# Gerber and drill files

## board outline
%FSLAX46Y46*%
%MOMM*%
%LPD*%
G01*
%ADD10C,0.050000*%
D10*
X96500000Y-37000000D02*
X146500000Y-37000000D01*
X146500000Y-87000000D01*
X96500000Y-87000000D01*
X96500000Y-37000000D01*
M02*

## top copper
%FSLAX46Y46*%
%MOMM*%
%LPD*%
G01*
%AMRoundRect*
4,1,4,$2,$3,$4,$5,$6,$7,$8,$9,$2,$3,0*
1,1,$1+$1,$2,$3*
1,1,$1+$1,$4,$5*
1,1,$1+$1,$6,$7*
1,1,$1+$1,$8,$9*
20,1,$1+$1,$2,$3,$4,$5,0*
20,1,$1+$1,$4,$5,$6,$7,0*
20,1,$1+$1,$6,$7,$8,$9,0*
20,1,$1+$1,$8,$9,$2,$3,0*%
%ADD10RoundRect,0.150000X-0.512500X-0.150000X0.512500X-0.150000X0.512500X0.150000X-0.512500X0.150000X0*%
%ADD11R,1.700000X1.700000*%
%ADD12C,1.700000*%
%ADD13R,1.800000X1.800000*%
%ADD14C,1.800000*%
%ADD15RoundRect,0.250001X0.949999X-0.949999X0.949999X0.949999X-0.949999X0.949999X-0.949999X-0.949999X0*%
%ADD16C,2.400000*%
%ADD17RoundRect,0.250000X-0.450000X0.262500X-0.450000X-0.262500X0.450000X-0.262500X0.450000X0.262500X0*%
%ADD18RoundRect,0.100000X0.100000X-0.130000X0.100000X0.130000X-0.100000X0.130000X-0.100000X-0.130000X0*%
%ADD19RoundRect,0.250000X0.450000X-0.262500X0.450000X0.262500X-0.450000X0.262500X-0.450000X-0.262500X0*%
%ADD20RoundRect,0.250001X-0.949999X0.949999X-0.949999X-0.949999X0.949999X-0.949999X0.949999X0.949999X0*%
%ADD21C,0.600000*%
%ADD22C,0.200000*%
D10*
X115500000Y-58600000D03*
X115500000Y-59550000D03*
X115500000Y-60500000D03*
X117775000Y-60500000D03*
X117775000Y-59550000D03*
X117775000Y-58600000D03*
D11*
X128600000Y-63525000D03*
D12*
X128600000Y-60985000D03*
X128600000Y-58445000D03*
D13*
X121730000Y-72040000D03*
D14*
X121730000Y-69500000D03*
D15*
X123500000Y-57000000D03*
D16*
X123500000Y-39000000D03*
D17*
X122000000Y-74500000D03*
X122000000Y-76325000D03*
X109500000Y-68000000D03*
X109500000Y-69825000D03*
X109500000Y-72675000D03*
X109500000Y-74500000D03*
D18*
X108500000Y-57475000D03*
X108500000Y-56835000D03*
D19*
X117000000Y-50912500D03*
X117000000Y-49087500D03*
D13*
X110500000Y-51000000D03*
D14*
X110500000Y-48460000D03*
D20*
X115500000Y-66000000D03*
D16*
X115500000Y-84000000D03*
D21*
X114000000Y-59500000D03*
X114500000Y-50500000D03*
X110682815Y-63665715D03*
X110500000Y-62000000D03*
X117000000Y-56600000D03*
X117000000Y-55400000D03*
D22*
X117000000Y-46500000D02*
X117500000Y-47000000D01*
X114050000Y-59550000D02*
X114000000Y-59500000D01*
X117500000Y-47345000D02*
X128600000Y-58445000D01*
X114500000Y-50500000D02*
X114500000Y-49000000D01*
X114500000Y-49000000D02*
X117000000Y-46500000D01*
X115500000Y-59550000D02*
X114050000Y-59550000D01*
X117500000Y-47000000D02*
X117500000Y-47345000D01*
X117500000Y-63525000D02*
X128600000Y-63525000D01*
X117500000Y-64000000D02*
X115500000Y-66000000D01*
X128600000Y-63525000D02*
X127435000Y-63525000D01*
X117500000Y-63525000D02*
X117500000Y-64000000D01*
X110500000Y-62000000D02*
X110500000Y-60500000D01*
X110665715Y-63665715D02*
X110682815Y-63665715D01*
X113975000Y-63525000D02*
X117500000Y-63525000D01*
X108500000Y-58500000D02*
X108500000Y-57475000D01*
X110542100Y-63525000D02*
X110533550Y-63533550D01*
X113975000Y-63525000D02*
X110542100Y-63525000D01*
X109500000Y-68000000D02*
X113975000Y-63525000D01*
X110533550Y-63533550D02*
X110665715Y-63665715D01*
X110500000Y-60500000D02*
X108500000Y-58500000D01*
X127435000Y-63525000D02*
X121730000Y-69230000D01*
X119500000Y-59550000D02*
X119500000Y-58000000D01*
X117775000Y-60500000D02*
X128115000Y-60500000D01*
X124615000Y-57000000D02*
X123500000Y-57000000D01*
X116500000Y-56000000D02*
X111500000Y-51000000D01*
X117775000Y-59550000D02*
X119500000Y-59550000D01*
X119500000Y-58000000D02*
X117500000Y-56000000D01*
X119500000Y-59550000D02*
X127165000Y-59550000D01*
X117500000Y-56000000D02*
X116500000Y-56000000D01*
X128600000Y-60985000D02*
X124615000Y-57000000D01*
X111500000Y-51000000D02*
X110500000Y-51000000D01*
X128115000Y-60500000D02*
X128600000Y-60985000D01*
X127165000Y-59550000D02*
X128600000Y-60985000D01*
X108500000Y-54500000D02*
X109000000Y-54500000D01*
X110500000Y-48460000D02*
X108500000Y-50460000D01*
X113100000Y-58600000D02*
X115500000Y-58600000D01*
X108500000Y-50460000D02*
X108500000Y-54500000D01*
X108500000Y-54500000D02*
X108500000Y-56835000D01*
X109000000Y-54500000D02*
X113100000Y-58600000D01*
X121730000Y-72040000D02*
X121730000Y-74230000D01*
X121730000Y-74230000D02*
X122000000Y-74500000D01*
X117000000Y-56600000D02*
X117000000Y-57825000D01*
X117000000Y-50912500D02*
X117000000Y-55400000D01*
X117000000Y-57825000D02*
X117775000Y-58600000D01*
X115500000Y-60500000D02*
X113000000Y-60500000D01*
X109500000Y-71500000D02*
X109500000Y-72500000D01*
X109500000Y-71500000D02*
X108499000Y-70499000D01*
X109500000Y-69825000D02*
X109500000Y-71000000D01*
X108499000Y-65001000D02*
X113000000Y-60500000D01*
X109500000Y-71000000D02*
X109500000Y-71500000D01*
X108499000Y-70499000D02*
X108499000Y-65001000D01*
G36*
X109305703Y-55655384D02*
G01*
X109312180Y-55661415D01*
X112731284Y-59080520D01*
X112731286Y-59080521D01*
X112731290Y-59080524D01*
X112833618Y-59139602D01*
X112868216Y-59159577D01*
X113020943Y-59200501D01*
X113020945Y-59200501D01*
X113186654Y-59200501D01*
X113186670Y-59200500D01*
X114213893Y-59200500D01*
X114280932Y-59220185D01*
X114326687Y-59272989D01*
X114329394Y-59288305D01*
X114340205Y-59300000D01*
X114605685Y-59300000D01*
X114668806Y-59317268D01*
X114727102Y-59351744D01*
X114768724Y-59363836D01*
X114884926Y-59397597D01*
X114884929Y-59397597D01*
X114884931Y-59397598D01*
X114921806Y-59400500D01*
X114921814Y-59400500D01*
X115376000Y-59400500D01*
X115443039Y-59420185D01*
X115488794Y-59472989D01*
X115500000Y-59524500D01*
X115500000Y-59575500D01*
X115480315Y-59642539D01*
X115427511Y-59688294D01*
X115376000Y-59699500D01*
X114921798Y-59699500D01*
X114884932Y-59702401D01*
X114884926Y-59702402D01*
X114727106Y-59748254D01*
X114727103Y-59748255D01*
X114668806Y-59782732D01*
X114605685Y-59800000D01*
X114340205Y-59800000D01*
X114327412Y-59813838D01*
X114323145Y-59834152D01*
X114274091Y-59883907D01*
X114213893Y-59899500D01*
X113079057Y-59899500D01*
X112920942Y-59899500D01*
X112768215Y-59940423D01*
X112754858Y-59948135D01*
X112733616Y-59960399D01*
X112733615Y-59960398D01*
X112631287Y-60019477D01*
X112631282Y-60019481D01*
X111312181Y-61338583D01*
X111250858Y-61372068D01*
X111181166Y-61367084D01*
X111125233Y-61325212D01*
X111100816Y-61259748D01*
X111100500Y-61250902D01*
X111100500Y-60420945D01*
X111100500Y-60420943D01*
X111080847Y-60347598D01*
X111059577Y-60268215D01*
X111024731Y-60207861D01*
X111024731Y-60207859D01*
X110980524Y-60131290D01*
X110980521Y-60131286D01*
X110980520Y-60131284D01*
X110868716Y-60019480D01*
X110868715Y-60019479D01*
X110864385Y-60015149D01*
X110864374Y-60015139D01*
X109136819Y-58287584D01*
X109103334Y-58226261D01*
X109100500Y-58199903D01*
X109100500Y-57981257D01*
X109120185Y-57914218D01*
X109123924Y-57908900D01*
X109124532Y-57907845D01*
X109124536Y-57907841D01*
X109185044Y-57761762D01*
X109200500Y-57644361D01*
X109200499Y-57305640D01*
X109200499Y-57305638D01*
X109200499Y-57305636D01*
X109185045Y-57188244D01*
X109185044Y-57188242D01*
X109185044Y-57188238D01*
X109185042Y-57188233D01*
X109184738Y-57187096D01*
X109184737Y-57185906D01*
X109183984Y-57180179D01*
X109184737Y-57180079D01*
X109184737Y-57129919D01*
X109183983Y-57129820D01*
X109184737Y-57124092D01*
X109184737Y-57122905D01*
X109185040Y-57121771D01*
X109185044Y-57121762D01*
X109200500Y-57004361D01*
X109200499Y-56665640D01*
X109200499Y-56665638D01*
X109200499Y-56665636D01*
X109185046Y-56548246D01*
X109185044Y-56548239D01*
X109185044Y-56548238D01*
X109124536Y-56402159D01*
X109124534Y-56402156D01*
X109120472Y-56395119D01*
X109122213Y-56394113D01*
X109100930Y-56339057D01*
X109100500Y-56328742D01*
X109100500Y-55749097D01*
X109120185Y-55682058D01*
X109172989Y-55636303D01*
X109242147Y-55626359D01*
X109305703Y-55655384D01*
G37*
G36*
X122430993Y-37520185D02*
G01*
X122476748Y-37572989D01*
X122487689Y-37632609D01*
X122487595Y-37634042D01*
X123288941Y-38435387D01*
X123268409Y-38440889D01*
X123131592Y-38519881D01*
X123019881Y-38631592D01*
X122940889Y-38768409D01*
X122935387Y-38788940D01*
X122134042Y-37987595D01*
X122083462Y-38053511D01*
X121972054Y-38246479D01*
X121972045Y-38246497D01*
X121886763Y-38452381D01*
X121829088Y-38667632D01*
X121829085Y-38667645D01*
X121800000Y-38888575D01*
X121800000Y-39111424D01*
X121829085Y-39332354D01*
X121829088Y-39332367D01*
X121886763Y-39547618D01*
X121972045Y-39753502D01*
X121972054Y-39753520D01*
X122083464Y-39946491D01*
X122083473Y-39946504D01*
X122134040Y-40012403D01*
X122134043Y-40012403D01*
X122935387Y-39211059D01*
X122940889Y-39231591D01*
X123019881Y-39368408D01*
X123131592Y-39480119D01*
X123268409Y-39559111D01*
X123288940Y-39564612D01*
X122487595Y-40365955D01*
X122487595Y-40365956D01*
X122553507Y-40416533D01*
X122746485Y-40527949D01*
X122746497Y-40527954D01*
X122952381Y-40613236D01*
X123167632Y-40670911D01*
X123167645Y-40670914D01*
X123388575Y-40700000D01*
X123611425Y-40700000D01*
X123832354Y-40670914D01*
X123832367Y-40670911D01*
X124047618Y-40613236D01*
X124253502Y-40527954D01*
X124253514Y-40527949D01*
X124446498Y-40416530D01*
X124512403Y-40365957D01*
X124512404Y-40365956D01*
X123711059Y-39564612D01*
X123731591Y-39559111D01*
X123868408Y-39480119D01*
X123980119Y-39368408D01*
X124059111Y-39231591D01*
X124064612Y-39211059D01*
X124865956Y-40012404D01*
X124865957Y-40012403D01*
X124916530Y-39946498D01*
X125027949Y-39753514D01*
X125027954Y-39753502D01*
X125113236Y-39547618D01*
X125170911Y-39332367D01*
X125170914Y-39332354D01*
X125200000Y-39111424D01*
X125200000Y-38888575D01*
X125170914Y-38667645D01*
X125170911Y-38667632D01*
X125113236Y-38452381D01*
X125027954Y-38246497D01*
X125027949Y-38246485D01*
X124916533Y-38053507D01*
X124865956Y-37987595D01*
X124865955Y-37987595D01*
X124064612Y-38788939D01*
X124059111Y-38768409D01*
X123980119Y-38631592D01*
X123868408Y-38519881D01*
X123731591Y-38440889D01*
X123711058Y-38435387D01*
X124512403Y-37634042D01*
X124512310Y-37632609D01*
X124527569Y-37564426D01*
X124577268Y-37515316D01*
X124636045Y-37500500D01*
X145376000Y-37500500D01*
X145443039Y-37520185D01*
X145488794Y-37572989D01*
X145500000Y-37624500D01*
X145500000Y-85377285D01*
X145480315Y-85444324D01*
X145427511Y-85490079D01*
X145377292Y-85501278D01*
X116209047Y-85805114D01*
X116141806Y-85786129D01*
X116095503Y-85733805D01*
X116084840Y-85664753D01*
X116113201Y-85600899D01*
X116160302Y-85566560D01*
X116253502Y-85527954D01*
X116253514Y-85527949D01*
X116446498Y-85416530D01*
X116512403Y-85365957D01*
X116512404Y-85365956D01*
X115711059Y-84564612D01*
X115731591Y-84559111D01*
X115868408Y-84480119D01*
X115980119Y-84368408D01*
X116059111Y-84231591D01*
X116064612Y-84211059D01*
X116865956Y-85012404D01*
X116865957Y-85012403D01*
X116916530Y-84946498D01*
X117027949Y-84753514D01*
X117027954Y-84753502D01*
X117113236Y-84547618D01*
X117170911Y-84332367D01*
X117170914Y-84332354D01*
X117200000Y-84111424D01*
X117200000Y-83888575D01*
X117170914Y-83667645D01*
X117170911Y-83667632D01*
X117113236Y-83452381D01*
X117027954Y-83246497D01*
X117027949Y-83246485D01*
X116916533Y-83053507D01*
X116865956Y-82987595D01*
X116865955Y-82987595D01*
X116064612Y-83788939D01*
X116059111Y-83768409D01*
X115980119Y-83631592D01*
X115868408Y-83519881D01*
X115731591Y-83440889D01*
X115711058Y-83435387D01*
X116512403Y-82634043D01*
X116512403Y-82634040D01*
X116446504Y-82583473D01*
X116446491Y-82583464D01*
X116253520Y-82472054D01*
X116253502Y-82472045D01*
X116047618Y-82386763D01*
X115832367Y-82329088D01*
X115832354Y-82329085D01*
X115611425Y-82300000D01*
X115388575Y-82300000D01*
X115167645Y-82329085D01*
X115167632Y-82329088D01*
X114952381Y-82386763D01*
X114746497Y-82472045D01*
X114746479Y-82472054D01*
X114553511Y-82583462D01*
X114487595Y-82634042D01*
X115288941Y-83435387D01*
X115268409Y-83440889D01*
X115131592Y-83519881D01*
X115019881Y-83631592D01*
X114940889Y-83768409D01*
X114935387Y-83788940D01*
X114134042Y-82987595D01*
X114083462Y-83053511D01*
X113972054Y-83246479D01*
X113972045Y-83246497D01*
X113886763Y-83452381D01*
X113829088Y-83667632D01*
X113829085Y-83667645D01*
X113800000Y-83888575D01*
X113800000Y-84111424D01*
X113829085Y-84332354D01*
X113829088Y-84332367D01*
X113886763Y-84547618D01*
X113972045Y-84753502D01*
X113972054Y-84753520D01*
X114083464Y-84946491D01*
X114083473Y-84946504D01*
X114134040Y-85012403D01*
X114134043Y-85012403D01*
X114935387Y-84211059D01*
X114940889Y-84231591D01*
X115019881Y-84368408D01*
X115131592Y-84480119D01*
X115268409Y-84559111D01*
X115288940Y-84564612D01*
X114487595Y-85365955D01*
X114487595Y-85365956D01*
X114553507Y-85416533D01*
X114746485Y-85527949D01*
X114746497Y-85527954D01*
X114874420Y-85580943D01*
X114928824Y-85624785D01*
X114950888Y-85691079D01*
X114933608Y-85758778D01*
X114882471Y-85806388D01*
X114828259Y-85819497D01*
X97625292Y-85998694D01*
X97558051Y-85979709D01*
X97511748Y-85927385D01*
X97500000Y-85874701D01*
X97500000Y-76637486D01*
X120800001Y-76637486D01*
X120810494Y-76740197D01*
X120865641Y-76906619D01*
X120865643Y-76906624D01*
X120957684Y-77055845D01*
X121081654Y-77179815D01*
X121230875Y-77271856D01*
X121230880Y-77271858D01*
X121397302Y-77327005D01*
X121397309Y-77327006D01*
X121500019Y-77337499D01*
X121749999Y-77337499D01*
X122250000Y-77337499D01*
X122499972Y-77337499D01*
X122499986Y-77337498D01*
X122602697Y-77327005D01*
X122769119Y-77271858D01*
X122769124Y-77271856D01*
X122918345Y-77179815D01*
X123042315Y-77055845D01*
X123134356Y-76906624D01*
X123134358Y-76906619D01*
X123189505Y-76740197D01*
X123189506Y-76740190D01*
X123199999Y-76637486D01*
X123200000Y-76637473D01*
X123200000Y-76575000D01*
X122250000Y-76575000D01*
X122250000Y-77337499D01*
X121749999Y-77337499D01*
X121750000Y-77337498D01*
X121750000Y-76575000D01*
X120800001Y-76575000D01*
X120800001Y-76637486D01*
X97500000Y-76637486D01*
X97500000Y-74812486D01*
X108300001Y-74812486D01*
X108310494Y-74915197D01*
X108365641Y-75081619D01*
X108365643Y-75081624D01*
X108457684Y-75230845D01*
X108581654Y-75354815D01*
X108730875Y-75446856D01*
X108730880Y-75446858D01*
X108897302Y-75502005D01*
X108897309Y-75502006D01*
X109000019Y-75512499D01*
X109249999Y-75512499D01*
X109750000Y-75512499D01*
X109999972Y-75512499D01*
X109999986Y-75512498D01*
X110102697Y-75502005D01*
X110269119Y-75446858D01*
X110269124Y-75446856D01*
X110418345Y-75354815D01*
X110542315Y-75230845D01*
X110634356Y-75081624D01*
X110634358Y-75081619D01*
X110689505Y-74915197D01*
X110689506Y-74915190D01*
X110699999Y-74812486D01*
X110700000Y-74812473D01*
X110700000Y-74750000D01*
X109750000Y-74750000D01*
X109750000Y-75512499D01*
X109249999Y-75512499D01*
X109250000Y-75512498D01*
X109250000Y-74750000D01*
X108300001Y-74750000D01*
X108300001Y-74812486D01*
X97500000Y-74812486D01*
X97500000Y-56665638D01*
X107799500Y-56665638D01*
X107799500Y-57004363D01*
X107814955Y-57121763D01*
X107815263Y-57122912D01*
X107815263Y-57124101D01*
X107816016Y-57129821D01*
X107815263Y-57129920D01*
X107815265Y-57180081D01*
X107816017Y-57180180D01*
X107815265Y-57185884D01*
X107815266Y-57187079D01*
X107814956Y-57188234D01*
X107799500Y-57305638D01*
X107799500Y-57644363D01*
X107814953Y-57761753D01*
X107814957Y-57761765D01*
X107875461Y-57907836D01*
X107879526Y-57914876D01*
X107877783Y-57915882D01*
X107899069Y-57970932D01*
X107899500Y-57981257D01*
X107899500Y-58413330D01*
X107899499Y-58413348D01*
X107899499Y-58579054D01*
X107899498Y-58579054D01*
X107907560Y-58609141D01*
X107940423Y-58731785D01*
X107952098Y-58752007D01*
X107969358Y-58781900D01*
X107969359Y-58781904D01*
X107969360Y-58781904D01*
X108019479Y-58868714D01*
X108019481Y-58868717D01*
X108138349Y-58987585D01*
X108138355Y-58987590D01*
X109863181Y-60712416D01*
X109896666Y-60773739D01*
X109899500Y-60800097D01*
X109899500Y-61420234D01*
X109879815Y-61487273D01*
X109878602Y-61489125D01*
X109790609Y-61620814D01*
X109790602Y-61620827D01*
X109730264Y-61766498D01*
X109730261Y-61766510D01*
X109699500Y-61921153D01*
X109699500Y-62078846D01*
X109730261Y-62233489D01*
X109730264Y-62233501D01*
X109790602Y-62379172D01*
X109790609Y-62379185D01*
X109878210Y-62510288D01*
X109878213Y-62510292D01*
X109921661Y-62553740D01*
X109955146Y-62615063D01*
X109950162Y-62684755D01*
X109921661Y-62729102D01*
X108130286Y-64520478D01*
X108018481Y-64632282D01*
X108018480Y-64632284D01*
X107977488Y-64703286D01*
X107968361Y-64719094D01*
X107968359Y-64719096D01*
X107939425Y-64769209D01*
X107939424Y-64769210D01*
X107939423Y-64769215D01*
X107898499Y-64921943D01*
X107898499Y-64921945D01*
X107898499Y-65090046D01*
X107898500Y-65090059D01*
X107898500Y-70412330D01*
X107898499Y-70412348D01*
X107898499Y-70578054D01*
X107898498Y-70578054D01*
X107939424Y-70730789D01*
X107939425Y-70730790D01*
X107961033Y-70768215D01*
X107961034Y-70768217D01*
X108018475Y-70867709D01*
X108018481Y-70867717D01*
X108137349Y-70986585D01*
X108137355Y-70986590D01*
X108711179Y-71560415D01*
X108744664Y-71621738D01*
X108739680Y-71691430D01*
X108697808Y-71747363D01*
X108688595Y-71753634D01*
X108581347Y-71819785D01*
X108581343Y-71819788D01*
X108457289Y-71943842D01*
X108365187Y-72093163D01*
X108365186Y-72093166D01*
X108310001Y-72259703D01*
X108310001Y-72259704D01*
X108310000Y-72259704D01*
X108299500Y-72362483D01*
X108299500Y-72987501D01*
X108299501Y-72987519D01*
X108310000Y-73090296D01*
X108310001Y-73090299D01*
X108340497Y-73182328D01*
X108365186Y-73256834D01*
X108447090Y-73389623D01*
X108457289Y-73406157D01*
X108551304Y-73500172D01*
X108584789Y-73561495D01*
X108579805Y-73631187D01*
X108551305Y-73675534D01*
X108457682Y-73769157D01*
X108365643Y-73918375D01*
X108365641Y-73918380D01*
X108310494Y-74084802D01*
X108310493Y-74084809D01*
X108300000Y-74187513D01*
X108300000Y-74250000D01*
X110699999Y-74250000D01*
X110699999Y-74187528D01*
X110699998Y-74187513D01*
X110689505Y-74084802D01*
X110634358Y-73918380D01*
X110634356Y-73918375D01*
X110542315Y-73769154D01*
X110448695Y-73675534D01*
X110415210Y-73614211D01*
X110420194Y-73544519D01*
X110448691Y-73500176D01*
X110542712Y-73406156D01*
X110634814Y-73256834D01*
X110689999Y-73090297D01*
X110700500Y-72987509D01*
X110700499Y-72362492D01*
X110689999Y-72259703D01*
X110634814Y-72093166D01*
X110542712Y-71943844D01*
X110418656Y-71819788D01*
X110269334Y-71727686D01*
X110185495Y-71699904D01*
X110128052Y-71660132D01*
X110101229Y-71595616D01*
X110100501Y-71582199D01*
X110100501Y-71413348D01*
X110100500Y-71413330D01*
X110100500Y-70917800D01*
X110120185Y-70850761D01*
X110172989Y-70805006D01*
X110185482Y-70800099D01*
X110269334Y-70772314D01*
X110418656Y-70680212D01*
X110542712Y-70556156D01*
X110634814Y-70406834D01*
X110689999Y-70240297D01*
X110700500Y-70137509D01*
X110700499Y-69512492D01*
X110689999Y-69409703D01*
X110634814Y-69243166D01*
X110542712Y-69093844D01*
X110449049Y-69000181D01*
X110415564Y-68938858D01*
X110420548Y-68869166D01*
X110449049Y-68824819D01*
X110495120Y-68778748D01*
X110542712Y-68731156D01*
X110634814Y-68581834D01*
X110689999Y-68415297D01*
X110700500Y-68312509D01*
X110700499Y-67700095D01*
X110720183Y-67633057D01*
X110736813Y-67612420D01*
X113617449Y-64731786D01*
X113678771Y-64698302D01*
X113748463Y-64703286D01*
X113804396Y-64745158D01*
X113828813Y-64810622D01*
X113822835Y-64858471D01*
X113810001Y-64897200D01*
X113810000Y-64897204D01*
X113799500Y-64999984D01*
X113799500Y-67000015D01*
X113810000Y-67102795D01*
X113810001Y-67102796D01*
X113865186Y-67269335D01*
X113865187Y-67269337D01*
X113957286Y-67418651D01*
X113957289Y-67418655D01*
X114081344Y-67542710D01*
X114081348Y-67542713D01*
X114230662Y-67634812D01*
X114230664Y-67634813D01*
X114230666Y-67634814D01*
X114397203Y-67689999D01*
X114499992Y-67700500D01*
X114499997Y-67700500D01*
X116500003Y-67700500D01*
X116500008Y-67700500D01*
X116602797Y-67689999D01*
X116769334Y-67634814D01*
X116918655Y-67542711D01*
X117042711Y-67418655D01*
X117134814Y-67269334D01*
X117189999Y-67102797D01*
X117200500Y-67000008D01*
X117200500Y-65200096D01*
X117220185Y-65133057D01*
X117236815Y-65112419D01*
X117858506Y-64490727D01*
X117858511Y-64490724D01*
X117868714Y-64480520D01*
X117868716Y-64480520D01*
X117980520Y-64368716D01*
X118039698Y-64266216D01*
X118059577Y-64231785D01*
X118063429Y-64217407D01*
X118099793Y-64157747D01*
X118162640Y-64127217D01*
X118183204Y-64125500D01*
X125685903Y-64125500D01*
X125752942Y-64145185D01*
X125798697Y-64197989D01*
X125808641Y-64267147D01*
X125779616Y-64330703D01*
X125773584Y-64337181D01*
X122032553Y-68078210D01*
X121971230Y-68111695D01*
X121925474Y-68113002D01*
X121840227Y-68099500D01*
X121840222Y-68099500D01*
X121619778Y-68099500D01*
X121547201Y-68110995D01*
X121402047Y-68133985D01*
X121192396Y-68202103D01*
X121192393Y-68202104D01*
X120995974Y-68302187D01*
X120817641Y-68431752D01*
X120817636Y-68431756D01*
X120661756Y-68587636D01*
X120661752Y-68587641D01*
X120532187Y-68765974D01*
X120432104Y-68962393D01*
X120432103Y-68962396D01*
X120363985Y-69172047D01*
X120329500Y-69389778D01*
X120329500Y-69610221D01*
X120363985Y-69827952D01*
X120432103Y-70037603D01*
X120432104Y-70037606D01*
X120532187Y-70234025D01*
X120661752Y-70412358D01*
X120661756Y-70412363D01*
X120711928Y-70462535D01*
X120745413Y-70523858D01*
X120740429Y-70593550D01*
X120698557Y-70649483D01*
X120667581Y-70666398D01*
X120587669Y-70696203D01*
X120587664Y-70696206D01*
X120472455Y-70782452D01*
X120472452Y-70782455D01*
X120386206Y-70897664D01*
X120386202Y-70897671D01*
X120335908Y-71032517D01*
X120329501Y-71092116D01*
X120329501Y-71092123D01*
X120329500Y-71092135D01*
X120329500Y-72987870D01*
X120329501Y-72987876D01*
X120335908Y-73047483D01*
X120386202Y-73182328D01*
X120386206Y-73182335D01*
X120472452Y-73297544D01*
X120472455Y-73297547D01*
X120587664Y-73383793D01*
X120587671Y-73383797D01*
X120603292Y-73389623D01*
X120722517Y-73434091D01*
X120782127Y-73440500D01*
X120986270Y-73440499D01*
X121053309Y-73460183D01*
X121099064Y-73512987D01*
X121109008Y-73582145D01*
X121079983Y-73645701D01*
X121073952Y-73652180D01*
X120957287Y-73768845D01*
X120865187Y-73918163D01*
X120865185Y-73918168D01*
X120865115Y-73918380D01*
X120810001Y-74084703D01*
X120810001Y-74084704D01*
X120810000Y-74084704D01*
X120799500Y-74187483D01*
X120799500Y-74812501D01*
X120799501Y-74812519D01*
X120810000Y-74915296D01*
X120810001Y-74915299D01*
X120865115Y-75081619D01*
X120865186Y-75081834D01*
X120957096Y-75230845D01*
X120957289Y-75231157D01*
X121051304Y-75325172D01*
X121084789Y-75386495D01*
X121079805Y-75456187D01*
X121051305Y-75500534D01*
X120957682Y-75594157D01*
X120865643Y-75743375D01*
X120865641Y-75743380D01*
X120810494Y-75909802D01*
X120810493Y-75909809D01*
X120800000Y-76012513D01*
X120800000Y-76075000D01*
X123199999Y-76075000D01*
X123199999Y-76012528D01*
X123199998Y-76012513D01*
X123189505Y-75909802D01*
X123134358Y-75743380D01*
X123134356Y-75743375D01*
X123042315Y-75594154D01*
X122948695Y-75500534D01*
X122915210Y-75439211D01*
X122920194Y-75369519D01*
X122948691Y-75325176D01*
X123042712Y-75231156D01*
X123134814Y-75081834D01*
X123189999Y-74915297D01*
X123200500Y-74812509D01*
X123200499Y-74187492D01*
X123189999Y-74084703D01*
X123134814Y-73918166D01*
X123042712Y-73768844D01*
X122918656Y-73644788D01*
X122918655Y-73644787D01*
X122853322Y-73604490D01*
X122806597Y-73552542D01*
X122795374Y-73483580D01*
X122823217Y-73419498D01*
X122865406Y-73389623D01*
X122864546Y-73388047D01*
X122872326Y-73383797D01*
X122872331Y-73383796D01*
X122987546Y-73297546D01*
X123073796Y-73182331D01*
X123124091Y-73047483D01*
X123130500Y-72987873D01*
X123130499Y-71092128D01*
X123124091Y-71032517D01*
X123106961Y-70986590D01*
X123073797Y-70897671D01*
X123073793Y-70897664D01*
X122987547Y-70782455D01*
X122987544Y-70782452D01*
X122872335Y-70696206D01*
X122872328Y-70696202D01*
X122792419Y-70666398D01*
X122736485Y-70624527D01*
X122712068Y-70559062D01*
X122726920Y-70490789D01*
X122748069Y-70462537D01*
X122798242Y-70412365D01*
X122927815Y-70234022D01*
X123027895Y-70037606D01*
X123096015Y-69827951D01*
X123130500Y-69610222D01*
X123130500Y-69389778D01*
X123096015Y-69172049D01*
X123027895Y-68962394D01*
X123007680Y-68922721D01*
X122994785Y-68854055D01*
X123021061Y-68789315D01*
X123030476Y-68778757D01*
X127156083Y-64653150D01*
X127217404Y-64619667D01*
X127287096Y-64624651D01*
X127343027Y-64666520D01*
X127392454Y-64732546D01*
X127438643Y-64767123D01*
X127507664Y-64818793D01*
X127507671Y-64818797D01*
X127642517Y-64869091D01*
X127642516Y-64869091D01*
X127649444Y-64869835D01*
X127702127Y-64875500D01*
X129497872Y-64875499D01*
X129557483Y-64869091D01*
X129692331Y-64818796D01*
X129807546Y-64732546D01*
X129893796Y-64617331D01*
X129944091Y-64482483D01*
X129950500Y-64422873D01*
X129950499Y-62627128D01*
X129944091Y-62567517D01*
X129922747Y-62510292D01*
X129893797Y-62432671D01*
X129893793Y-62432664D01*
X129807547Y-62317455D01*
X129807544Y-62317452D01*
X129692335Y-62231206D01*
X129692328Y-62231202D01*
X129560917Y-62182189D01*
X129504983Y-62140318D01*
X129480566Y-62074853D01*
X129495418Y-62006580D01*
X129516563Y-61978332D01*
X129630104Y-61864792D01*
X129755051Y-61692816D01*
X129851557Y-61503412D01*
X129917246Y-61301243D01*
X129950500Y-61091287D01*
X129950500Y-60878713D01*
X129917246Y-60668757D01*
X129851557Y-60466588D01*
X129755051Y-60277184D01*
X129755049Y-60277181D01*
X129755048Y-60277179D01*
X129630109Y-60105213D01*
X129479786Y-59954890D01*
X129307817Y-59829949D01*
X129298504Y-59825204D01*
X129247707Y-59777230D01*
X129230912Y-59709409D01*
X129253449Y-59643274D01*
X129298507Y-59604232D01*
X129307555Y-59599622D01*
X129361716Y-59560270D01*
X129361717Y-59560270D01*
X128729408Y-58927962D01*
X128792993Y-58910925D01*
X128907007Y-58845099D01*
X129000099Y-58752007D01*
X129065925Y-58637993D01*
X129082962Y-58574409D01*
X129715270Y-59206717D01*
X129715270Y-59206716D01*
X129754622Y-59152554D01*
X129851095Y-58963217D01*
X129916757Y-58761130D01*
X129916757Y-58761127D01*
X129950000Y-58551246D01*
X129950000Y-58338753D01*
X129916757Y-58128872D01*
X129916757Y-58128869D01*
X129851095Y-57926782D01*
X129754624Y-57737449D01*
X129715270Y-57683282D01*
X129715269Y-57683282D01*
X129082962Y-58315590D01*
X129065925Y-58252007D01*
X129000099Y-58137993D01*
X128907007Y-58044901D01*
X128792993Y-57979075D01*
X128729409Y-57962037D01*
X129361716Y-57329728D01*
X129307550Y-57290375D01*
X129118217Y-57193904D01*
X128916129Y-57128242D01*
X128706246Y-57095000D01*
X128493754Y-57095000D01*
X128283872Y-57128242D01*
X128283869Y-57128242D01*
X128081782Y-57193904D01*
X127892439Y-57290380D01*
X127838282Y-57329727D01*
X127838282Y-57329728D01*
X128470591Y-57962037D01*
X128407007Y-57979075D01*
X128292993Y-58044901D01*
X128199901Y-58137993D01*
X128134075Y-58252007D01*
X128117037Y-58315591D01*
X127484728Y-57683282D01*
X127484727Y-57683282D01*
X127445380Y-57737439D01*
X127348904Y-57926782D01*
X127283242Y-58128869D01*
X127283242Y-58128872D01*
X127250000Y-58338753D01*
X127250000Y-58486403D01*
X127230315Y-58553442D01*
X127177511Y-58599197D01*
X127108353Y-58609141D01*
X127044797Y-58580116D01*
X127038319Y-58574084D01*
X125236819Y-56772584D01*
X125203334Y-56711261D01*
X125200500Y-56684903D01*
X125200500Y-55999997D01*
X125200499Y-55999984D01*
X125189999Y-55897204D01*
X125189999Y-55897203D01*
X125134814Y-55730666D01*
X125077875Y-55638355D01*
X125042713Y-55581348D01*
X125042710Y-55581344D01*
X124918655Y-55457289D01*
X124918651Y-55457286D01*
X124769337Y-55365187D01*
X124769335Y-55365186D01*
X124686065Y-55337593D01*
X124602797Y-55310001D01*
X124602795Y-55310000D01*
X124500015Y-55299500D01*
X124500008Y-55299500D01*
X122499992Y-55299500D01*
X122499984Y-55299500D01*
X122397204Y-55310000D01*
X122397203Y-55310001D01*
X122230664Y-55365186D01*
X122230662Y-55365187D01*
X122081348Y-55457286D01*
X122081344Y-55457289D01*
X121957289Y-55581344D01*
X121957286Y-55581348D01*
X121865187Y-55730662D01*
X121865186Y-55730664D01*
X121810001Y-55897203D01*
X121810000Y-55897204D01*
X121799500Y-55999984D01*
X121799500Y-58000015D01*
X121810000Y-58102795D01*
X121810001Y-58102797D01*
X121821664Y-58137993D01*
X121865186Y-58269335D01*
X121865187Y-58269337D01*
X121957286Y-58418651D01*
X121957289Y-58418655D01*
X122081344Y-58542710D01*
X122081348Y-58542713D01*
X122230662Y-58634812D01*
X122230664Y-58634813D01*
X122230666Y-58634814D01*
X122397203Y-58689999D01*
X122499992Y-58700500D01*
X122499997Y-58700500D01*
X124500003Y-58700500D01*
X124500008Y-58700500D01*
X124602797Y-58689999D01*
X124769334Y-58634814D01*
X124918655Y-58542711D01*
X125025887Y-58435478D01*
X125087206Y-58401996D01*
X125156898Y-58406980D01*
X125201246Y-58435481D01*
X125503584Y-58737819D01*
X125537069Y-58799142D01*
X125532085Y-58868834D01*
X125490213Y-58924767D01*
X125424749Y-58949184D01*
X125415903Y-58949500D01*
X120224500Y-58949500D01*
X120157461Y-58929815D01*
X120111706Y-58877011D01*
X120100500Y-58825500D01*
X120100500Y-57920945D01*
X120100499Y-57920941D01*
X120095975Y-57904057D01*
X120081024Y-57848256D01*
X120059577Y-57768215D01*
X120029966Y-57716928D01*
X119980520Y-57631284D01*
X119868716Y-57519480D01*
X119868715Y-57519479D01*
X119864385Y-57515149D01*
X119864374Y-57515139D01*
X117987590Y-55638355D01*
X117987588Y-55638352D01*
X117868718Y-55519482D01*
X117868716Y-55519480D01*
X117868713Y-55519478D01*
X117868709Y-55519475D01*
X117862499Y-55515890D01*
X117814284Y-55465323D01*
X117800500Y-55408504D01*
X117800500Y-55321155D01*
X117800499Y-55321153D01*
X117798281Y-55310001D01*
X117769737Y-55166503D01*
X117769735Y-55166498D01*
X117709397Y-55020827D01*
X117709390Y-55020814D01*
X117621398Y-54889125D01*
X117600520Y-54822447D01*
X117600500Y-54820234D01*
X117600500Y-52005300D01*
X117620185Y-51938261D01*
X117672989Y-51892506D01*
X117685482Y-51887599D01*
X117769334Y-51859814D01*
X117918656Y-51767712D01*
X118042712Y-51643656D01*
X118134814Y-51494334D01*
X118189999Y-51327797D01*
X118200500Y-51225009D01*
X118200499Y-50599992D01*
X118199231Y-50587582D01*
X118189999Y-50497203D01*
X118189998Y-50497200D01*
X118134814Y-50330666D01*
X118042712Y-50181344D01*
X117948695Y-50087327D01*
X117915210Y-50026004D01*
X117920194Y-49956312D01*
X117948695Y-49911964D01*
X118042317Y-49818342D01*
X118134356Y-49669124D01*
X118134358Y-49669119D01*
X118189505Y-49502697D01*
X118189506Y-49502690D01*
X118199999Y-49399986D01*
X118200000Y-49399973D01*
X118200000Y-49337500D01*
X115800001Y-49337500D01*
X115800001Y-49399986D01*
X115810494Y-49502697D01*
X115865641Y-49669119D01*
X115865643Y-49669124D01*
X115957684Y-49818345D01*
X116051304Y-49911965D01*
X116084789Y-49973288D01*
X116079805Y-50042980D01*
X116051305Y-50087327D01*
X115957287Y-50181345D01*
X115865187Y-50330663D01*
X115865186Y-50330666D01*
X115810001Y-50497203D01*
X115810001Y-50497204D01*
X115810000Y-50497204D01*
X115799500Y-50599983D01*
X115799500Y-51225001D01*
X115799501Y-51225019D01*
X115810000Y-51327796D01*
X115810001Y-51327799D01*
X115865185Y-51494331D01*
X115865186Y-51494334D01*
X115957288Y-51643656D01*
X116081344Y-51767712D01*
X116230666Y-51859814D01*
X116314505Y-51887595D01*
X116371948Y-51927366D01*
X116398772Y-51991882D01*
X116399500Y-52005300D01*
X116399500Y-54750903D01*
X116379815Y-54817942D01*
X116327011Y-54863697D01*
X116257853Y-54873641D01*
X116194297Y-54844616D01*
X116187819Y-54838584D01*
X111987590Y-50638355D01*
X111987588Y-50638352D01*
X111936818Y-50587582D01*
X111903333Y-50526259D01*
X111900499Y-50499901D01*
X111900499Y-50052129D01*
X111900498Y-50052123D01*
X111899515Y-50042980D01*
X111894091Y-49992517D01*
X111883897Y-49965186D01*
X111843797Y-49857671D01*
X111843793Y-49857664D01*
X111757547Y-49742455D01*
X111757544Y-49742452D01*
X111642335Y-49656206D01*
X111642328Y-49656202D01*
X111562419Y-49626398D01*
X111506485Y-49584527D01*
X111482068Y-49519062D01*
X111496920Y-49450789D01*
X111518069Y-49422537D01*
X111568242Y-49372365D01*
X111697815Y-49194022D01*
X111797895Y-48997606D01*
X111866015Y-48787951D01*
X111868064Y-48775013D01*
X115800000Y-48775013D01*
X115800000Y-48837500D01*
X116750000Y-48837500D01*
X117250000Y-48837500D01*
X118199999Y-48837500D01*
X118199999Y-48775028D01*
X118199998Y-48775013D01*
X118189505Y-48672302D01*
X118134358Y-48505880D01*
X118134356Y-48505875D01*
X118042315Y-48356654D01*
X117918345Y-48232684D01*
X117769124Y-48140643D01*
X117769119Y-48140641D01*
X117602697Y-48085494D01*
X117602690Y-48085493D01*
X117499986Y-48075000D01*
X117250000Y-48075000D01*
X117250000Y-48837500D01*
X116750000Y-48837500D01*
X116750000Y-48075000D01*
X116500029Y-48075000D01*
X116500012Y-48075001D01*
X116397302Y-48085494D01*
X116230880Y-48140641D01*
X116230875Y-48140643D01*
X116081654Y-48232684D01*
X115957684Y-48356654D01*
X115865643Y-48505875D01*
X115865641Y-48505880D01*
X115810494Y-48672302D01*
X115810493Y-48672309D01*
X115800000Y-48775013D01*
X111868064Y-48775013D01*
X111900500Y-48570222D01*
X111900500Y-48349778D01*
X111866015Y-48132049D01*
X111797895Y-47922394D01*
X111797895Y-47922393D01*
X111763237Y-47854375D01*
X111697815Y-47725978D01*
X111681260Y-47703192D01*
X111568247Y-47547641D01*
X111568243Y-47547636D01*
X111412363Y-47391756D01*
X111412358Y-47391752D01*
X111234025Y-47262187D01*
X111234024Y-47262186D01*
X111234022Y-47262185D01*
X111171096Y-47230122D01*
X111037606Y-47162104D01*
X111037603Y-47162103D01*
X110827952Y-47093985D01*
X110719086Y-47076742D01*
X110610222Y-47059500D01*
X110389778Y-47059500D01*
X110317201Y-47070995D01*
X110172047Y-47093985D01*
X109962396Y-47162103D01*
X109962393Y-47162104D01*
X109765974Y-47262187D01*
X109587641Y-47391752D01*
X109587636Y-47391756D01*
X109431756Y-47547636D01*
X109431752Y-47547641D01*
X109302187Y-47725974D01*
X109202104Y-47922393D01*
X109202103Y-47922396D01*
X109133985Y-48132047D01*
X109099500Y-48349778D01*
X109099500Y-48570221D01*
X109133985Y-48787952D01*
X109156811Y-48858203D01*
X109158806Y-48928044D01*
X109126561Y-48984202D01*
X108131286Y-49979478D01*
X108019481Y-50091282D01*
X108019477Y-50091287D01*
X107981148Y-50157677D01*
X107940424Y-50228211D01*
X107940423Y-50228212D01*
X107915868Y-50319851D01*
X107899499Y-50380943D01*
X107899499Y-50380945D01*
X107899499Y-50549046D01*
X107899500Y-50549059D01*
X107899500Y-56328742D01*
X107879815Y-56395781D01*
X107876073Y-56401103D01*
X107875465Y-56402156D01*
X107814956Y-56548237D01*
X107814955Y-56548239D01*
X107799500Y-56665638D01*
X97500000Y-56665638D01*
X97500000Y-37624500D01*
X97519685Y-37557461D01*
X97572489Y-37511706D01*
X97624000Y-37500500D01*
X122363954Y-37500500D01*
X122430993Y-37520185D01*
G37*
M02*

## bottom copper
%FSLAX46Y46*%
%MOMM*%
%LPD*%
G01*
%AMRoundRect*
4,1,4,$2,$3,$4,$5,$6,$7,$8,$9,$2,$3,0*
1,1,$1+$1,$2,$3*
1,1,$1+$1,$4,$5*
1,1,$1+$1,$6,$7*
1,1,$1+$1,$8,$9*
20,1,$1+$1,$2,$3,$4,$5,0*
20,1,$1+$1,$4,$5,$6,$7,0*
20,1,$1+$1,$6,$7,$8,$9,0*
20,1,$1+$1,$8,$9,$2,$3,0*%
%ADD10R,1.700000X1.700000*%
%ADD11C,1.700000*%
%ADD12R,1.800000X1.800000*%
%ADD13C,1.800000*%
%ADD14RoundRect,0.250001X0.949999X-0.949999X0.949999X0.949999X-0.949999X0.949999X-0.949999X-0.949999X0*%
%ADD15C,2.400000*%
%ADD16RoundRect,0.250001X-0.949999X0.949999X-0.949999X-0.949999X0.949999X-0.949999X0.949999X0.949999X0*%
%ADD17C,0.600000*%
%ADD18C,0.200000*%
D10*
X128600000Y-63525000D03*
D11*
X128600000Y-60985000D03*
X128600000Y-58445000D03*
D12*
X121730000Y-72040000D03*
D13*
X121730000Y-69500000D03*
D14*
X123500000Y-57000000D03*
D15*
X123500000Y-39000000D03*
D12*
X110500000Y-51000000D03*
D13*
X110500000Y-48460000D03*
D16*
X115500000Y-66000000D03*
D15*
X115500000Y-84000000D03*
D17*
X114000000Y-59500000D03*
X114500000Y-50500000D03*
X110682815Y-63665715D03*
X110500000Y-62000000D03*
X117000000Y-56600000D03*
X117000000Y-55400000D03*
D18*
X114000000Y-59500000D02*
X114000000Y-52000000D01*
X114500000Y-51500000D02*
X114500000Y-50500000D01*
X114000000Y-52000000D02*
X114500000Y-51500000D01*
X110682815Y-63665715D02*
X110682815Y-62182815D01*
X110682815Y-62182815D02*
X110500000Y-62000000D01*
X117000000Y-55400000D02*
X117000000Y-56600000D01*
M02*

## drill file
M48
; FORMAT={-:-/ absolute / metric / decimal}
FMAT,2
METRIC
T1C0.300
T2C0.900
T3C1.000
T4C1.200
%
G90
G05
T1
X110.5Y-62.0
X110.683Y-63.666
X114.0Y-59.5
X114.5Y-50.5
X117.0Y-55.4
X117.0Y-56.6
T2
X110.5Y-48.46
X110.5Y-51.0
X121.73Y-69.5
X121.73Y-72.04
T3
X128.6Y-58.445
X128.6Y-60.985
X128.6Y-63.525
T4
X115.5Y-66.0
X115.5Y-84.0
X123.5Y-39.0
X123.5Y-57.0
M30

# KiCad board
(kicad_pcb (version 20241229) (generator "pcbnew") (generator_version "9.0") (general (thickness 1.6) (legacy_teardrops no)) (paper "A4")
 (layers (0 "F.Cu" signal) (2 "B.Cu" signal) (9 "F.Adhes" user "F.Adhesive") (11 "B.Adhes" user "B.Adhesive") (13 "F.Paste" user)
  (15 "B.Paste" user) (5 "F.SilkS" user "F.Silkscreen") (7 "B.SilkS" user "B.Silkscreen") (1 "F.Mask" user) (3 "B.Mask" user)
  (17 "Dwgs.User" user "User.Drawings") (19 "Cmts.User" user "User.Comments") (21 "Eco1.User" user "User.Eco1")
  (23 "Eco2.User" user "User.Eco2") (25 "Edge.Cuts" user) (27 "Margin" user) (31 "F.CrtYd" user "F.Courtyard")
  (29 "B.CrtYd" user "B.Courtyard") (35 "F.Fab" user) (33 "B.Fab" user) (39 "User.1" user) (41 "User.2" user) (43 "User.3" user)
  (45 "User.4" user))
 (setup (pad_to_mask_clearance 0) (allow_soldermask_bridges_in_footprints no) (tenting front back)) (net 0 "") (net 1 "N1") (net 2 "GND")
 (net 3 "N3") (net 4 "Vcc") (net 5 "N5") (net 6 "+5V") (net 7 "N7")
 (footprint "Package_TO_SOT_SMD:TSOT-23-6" (layer "F.Cu") (at 116.6375 59.55)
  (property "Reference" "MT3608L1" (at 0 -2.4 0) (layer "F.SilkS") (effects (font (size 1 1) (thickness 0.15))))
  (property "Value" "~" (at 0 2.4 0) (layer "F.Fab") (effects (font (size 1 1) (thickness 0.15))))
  (pad "1" smd roundrect (at -1.1375 -0.95) (size 1.325 0.6) (layers "F.Cu" "F.Mask" "F.Paste") (roundrect_rratio 0.25) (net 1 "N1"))
  (pad "2" smd roundrect (at -1.1375 0) (size 1.325 0.6) (layers "F.Cu" "F.Mask" "F.Paste") (roundrect_rratio 0.25) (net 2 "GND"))
  (pad "3" smd roundrect (at -1.1375 0.95) (size 1.325 0.6) (layers "F.Cu" "F.Mask" "F.Paste") (roundrect_rratio 0.25) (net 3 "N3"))
  (pad "4" smd roundrect (at 1.1375 0.95) (size 1.325 0.6) (layers "F.Cu" "F.Mask" "F.Paste") (roundrect_rratio 0.25) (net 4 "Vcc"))
  (pad "5" smd roundrect (at 1.1375 0) (size 1.325 0.6) (layers "F.Cu" "F.Mask" "F.Paste") (roundrect_rratio 0.25) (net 4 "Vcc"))
  (pad "6" smd roundrect (at 1.1375 -0.95) (size 1.325 0.6) (layers "F.Cu" "F.Mask" "F.Paste") (roundrect_rratio 0.25) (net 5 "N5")))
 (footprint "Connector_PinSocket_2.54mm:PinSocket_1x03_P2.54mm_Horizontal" (layer "F.Cu") (at 128.6 63.525 180)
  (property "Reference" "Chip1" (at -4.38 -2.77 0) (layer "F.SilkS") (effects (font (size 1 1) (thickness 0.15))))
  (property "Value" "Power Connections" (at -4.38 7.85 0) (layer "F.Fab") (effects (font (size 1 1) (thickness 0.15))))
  (pad "1" thru_hole rect (at 0 0 180) (size 1.7 1.7) (drill 1) (layers "*.Cu" "*.Mask") (remove_unused_layers no) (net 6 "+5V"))
  (pad "2" thru_hole circle (at 0 2.54 180) (size 1.7 1.7) (drill 1) (layers "*.Cu" "*.Mask") (remove_unused_layers no) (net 4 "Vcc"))
  (pad "3" thru_hole circle (at 0 5.08 180) (size 1.7 1.7) (drill 1) (layers "*.Cu" "*.Mask") (remove_unused_layers no) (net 2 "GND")))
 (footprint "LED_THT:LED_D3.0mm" (layer "F.Cu") (at 121.73 72.04 90)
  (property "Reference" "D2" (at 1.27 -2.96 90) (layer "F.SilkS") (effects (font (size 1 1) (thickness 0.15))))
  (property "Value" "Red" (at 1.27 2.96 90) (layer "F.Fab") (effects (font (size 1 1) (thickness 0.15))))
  (pad "1" thru_hole rect (at 0 0 90) (size 1.8 1.8) (drill 0.9) (layers "*.Cu" "*.Mask") (remove_unused_layers no) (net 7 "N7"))
  (pad "2" thru_hole circle (at 2.54 0 90) (size 1.8 1.8) (drill 0.9) (layers "*.Cu" "*.Mask") (remove_unused_layers no) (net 6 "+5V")))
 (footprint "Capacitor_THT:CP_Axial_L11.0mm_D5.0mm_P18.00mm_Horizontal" (layer "F.Cu") (at 123.5 57 90)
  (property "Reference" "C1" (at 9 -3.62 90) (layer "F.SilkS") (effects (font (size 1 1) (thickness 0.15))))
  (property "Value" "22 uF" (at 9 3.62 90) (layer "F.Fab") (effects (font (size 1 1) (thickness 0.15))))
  (pad "1" thru_hole roundrect (at 0 0 90) (size 2.4 2.4) (drill 1.2) (layers "*.Cu" "*.Mask") (remove_unused_layers no)
   (roundrect_rratio 0.104167) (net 4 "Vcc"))
  (pad "2" thru_hole circle (at 18 0 90) (size 2.4 2.4) (drill 1.2) (layers "*.Cu" "*.Mask") (remove_unused_layers no) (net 2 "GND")))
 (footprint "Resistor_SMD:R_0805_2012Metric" (layer "F.Cu") (at 122 75.4125 -90)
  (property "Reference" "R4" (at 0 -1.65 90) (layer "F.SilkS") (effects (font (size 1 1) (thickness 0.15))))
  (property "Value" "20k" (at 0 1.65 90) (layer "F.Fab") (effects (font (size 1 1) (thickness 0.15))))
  (pad "1" smd roundrect (at -0.9125 0 270) (size 1.025 1.4) (layers "F.Cu" "F.Mask" "F.Paste") (roundrect_rratio 0.243902) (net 7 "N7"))
  (pad "2" smd roundrect (at 0.9125 0 270) (size 1.025 1.4) (layers "F.Cu" "F.Mask" "F.Paste") (roundrect_rratio 0.243902) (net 2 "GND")))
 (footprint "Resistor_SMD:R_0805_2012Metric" (layer "F.Cu") (at 109.5 68.9125 -90)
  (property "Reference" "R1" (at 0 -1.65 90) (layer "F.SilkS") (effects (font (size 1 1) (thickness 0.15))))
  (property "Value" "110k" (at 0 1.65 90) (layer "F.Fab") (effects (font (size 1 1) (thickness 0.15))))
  (pad "1" smd roundrect (at -0.9125 0 270) (size 1.025 1.4) (layers "F.Cu" "F.Mask" "F.Paste") (roundrect_rratio 0.243902) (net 6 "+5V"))
  (pad "2" smd roundrect (at 0.9125 0 270) (size 1.025 1.4) (layers "F.Cu" "F.Mask" "F.Paste") (roundrect_rratio 0.243902) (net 3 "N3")))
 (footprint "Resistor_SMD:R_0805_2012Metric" (layer "F.Cu") (at 109.5 73.5875 -90)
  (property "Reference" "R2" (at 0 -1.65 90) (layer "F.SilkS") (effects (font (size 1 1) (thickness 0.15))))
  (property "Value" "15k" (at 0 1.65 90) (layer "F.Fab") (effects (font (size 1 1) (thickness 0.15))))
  (pad "1" smd roundrect (at -0.9125 0 270) (size 1.025 1.4) (layers "F.Cu" "F.Mask" "F.Paste") (roundrect_rratio 0.243902) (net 3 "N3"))
  (pad "2" smd roundrect (at 0.9125 0 270) (size 1.025 1.4) (layers "F.Cu" "F.Mask" "F.Paste") (roundrect_rratio 0.243902) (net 2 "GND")))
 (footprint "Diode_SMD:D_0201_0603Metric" (layer "F.Cu") (at 108.5 57.155 90)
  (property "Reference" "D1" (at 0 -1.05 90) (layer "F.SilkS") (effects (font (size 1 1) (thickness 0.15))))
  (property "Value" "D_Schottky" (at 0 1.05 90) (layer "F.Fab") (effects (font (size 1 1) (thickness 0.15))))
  (pad "" smd roundrect (at -0.345 0 90) (size 0.318 0.36) (layers "F.Paste") (roundrect_rratio 0.25))
  (pad "" smd roundrect (at 0.345 0 90) (size 0.318 0.36) (layers "F.Paste") (roundrect_rratio 0.25))
  (pad "1" smd roundrect (at -0.32 0 90) (size 0.46 0.4) (layers "F.Cu" "F.Mask") (roundrect_rratio 0.25) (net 6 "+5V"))
  (pad "2" smd roundrect (at 0.32 0 90) (size 0.46 0.4) (layers "F.Cu" "F.Mask") (roundrect_rratio 0.25) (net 1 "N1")))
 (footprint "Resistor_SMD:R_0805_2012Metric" (layer "F.Cu") (at 117 50 90)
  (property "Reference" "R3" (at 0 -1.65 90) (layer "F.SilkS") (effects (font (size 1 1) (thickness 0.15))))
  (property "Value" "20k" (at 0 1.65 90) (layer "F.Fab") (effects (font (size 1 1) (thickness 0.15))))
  (pad "1" smd roundrect (at -0.9125 0 90) (size 1.025 1.4) (layers "F.Cu" "F.Mask" "F.Paste") (roundrect_rratio 0.243902) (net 5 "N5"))
  (pad "2" smd roundrect (at 0.9125 0 90) (size 1.025 1.4) (layers "F.Cu" "F.Mask" "F.Paste") (roundrect_rratio 0.243902) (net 2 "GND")))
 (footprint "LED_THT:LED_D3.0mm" (layer "F.Cu") (at 110.5 51 90)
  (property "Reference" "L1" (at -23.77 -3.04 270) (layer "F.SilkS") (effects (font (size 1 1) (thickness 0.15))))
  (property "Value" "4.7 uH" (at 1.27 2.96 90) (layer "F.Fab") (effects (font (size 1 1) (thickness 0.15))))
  (pad "1" thru_hole rect (at 0 0 90) (size 1.8 1.8) (drill 0.9) (layers "*.Cu" "*.Mask") (remove_unused_layers no) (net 4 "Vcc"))
  (pad "2" thru_hole circle (at 2.54 0 90) (size 1.8 1.8) (drill 0.9) (layers "*.Cu" "*.Mask") (remove_unused_layers no) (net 1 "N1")))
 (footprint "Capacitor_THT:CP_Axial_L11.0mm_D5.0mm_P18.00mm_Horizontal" (layer "F.Cu") (at 115.5 66 -90)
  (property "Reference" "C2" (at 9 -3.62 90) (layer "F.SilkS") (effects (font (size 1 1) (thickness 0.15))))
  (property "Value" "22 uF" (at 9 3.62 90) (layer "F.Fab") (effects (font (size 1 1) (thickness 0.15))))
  (pad "1" thru_hole roundrect (at 0 0 270) (size 2.4 2.4) (drill 1.2) (layers "*.Cu" "*.Mask") (remove_unused_layers no)
   (roundrect_rratio 0.104167) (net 6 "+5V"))
  (pad "2" thru_hole circle (at 18 0 270) (size 2.4 2.4) (drill 1.2) (layers "*.Cu" "*.Mask") (remove_unused_layers no) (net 2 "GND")))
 (gr_rect (start 96.5 37) (end 146.5 87) (stroke (width 0.05) (type default)) (fill no) (layer "Edge.Cuts"))
 (segment (start 117 46.5) (end 117.5 47) (width 0.2) (layer "F.Cu") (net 2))
 (segment (start 114.05 59.55) (end 114 59.5) (width 0.2) (layer "F.Cu") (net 2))
 (segment (start 117.5 47.345) (end 128.6 58.445) (width 0.2) (layer "F.Cu") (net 2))
 (segment (start 114.5 50.5) (end 114.5 49) (width 0.2) (layer "F.Cu") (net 2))
 (segment (start 114.5 49) (end 117 46.5) (width 0.2) (layer "F.Cu") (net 2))
 (segment (start 115.5 59.55) (end 114.05 59.55) (width 0.2) (layer "F.Cu") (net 2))
 (segment (start 117.5 47) (end 117.5 47.345) (width 0.2) (layer "F.Cu") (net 2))
 (via (at 114 59.5) (size 0.6) (drill 0.3) (layers "F.Cu" "B.Cu") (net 2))
 (via (at 114.5 50.5) (size 0.6) (drill 0.3) (layers "F.Cu" "B.Cu") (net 2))
 (segment (start 114 59.5) (end 114 52) (width 0.2) (layer "B.Cu") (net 2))
 (segment (start 114.5 51.5) (end 114.5 50.5) (width 0.2) (layer "B.Cu") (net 2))
 (segment (start 114 52) (end 114.5 51.5) (width 0.2) (layer "B.Cu") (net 2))
 (segment (start 117.5 63.525) (end 128.6 63.525) (width 0.2) (layer "F.Cu") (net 6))
 (segment (start 117.5 64) (end 115.5 66) (width 0.2) (layer "F.Cu") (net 6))
 (segment (start 128.6 63.525) (end 127.435 63.525) (width 0.2) (layer "F.Cu") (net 6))
 (segment (start 117.5 63.525) (end 117.5 64) (width 0.2) (layer "F.Cu") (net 6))
 (segment (start 110.5 62) (end 110.5 60.5) (width 0.2) (layer "F.Cu") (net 6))
 (segment (start 110.665715 63.665715) (end 110.682815 63.665715) (width 0.2) (layer "F.Cu") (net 6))
 (segment (start 113.975 63.525) (end 117.5 63.525) (width 0.2) (layer "F.Cu") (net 6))
 (segment (start 108.5 58.5) (end 108.5 57.475) (width 0.2) (layer "F.Cu") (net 6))
 (segment (start 110.5421 63.525) (end 110.53355 63.53355) (width 0.2) (layer "F.Cu") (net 6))
 (segment (start 113.975 63.525) (end 110.5421 63.525) (width 0.2) (layer "F.Cu") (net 6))
 (segment (start 109.5 68) (end 113.975 63.525) (width 0.2) (layer "F.Cu") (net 6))
 (segment (start 110.53355 63.53355) (end 110.665715 63.665715) (width 0.2) (layer "F.Cu") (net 6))
 (segment (start 110.5 60.5) (end 108.5 58.5) (width 0.2) (layer "F.Cu") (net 6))
 (segment (start 127.435 63.525) (end 121.73 69.23) (width 0.2) (layer "F.Cu") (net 6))
 (via (at 110.682815 63.665715) (size 0.6) (drill 0.3) (layers "F.Cu" "B.Cu") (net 6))
 (via (at 110.5 62) (size 0.6) (drill 0.3) (layers "F.Cu" "B.Cu") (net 6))
 (segment (start 110.682815 63.665715) (end 110.682815 62.182815) (width 0.2) (layer "B.Cu") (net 6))
 (segment (start 110.682815 62.182815) (end 110.5 62) (width 0.2) (layer "B.Cu") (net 6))
 (segment (start 119.5 59.55) (end 119.5 58) (width 0.2) (layer "F.Cu") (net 4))
 (segment (start 117.775 60.5) (end 128.115 60.5) (width 0.2) (layer "F.Cu") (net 4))
 (segment (start 124.615 57) (end 123.5 57) (width 0.2) (layer "F.Cu") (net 4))
 (segment (start 116.5 56) (end 111.5 51) (width 0.2) (layer "F.Cu") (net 4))
 (segment (start 117.775 59.55) (end 119.5 59.55) (width 0.2) (layer "F.Cu") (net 4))
 (segment (start 119.5 58) (end 117.5 56) (width 0.2) (layer "F.Cu") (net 4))
 (segment (start 119.5 59.55) (end 127.165 59.55) (width 0.2) (layer "F.Cu") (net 4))
 (segment (start 117.5 56) (end 116.5 56) (width 0.2) (layer "F.Cu") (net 4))
 (segment (start 128.6 60.985) (end 124.615 57) (width 0.2) (layer "F.Cu") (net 4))
 (segment (start 111.5 51) (end 110.5 51) (width 0.2) (layer "F.Cu") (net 4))
 (segment (start 128.115 60.5) (end 128.6 60.985) (width 0.2) (layer "F.Cu") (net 4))
 (segment (start 127.165 59.55) (end 128.6 60.985) (width 0.2) (layer "F.Cu") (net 4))
 (segment (start 108.5 54.5) (end 109 54.5) (width 0.2) (layer "F.Cu") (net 1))
 (segment (start 110.5 48.46) (end 108.5 50.46) (width 0.2) (layer "F.Cu") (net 1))
 (segment (start 113.1 58.6) (end 115.5 58.6) (width 0.2) (layer "F.Cu") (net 1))
 (segment (start 108.5 50.46) (end 108.5 54.5) (width 0.2) (layer "F.Cu") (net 1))
 (segment (start 108.5 54.5) (end 108.5 56.835) (width 0.2) (layer "F.Cu") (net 1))
 (segment (start 109 54.5) (end 113.1 58.6) (width 0.2) (layer "F.Cu") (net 1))
 (segment (start 121.73 72.04) (end 121.73 74.23) (width 0.2) (layer "F.Cu") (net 7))
 (segment (start 121.73 74.23) (end 122 74.5) (width 0.2) (layer "F.Cu") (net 7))
 (segment (start 117 56.6) (end 117 57.825) (width 0.2) (layer "F.Cu") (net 5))
 (segment (start 117 50.9125) (end 117 55.4) (width 0.2) (layer "F.Cu") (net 5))
 (segment (start 117 57.825) (end 117.775 58.6) (width 0.2) (layer "F.Cu") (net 5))
 (via (at 117 56.6) (size 0.6) (drill 0.3) (layers "F.Cu" "B.Cu") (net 5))
 (via (at 117 55.4) (size 0.6) (drill 0.3) (layers "F.Cu" "B.Cu") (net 5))
 (segment (start 117 55.4) (end 117 56.6) (width 0.2) (layer "B.Cu") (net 5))
 (segment (start 115.5 60.5) (end 113 60.5) (width 0.2) (layer "F.Cu") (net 3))
 (segment (start 109.5 71.5) (end 109.5 72.5) (width 0.2) (layer "F.Cu") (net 3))
 (segment (start 109.5 71.5) (end 108.499 70.499) (width 0.2) (layer "F.Cu") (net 3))
 (segment (start 109.5 69.825) (end 109.5 71) (width 0.2) (layer "F.Cu") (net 3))
 (segment (start 108.499 65.001) (end 113 60.5) (width 0.2) (layer "F.Cu") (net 3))
 (segment (start 109.5 71) (end 109.5 71.5) (width 0.2) (layer "F.Cu") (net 3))
 (segment (start 108.499 70.499) (end 108.499 65.001) (width 0.2) (layer "F.Cu") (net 3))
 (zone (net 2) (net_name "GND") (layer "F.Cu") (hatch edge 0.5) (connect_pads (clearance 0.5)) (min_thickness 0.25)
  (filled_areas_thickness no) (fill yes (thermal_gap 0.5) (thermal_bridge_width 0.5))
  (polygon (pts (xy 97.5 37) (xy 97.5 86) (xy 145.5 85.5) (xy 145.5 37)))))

